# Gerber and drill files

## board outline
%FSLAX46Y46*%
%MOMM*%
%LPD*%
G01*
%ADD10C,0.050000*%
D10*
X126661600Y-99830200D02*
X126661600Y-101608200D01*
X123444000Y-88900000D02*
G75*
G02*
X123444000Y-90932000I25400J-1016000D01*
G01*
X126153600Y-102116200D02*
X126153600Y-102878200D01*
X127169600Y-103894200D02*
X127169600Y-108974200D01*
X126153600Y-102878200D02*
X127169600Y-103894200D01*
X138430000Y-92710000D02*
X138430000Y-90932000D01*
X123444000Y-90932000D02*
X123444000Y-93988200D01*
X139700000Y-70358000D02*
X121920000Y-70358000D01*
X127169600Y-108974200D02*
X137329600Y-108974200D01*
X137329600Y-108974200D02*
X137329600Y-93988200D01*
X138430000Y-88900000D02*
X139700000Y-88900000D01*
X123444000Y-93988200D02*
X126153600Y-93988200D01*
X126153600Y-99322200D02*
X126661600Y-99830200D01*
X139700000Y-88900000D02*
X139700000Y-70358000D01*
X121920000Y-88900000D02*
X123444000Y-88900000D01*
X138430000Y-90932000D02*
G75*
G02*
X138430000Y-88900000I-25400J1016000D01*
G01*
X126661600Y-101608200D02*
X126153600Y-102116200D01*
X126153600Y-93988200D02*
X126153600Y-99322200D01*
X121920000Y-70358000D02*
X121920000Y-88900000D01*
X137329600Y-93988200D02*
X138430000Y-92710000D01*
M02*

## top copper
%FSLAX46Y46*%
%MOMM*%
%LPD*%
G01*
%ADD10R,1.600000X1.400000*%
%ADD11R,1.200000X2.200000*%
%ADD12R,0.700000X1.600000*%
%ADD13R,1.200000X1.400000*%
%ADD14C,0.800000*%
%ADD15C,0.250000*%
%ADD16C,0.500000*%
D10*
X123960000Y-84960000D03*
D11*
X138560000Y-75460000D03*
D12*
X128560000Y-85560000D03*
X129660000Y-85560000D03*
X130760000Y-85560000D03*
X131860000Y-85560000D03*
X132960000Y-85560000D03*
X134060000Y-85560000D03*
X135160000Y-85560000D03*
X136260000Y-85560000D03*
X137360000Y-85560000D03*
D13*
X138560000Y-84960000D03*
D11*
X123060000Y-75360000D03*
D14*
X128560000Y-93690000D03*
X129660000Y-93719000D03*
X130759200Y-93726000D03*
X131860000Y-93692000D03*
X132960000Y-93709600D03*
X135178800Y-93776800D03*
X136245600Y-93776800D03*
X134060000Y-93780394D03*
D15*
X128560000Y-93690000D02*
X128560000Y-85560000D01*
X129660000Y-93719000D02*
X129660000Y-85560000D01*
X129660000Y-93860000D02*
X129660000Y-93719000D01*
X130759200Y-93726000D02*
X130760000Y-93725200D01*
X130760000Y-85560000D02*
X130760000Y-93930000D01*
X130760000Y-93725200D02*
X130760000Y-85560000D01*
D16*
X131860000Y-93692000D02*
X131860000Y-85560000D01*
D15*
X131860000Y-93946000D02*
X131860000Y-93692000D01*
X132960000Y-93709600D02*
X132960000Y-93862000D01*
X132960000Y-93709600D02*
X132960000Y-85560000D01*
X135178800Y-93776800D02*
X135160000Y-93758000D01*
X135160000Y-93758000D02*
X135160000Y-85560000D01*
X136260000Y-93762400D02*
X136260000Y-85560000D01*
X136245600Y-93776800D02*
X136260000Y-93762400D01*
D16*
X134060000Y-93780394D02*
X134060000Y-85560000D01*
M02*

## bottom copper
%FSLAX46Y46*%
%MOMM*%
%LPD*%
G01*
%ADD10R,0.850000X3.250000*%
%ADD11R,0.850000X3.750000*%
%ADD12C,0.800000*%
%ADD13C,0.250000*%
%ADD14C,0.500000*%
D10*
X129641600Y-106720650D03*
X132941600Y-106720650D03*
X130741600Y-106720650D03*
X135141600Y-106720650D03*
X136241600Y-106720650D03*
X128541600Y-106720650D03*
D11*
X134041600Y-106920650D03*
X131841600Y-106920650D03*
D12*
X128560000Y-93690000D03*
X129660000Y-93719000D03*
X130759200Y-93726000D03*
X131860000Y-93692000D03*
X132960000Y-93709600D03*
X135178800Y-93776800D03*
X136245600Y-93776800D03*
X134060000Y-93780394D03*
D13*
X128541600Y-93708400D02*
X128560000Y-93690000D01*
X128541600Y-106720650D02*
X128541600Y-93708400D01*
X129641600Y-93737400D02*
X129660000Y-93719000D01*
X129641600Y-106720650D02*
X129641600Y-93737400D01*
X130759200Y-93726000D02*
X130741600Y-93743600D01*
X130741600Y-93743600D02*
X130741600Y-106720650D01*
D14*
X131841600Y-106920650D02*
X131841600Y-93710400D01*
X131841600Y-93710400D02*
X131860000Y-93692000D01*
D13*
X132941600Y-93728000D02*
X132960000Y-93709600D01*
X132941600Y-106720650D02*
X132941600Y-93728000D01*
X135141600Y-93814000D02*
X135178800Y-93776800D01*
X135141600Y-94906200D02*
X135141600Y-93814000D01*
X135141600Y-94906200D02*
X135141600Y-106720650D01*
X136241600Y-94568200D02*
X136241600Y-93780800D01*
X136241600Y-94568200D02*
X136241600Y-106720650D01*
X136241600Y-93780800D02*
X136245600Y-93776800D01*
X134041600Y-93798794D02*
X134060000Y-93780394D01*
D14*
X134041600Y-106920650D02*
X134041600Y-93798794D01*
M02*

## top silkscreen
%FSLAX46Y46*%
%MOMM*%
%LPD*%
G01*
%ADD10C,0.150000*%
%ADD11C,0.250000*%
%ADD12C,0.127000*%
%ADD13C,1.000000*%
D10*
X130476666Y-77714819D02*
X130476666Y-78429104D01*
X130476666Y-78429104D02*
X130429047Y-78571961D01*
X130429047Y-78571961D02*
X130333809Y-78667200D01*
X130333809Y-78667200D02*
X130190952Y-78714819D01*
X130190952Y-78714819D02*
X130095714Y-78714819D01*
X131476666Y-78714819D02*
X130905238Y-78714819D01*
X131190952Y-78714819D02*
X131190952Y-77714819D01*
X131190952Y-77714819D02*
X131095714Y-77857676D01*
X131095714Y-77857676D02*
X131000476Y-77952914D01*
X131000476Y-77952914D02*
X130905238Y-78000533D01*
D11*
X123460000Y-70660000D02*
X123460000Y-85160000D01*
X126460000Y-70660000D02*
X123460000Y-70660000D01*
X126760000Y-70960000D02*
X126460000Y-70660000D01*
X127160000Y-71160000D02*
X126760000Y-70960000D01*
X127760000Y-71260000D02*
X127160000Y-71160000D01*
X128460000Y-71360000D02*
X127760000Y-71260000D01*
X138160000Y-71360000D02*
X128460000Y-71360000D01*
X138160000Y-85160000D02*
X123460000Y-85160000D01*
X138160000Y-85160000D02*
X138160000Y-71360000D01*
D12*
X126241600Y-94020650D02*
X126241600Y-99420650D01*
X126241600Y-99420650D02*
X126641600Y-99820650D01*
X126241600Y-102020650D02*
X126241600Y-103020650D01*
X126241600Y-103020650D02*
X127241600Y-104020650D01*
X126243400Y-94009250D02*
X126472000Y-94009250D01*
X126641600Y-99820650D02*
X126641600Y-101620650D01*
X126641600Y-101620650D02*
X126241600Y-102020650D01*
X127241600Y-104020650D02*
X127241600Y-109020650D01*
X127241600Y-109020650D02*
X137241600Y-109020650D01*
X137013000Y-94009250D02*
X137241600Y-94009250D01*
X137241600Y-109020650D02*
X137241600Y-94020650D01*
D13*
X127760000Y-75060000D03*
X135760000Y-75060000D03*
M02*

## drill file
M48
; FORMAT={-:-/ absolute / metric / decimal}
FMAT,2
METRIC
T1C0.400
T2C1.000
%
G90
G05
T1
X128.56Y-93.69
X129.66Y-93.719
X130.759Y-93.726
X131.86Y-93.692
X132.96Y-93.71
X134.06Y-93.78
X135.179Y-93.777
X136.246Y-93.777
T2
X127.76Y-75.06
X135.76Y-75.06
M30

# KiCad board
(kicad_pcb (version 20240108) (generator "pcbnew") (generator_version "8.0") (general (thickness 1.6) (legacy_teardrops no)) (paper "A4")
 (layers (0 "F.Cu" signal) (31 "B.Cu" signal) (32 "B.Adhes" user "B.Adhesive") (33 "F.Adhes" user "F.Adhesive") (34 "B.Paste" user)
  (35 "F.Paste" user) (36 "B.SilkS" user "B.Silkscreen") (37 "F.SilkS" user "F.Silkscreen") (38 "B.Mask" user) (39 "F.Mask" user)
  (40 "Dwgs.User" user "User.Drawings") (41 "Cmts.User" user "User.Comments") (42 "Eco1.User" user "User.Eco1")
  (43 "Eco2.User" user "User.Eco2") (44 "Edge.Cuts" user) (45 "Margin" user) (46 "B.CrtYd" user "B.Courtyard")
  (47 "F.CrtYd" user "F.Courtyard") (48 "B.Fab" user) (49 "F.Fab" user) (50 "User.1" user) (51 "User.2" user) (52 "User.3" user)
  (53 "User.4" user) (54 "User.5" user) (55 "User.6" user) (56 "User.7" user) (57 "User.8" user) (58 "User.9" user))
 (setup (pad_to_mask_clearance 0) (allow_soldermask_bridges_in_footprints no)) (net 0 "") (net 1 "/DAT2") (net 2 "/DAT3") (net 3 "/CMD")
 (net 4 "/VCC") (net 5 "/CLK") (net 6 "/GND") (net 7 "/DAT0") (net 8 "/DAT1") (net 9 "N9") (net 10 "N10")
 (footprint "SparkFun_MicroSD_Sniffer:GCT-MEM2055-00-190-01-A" (layer "F.Cu") (at 130.81 86.36)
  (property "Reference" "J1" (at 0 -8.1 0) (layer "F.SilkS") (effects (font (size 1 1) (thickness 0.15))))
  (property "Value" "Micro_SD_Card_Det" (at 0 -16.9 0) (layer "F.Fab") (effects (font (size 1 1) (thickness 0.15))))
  (fp_line (start -7.35 -15.7) (end -7.35 -1.2) (stroke (width 0.25) (type solid)) (layer "F.SilkS"))
  (fp_line (start -4.35 -15.7) (end -7.35 -15.7) (stroke (width 0.25) (type solid)) (layer "F.SilkS"))
  (fp_line (start -4.05 -15.4) (end -4.35 -15.7) (stroke (width 0.25) (type solid)) (layer "F.SilkS"))
  (fp_line (start -3.65 -15.2) (end -4.05 -15.4) (stroke (width 0.25) (type solid)) (layer "F.SilkS"))
  (fp_line (start -3.05 -15.1) (end -3.65 -15.2) (stroke (width 0.25) (type solid)) (layer "F.SilkS"))
  (fp_line (start -2.35 -15) (end -3.05 -15.1) (stroke (width 0.25) (type solid)) (layer "F.SilkS"))
  (fp_line (start 7.35 -15) (end -2.35 -15) (stroke (width 0.25) (type solid)) (layer "F.SilkS"))
  (fp_line (start 7.35 -1.2) (end -7.35 -1.2) (stroke (width 0.25) (type solid)) (layer "F.SilkS"))
  (fp_line (start 7.35 -1.2) (end 7.35 -15) (stroke (width 0.25) (type solid)) (layer "F.SilkS"))
  (pad "" smd rect (at -6.85 -1.4) (size 1.6 1.4) (layers "F.Cu" "F.Paste" "F.Mask"))
  (pad "" np_thru_hole circle (at -3.05 -11.3 180) (size 1 1) (drill 1) (layers "*.Cu" "*.Mask" "F.SilkS"))
  (pad "" np_thru_hole circle (at 4.95 -11.3 180) (size 1 1) (drill 1) (layers "*.Cu" "*.Mask" "F.SilkS"))
  (pad "" smd rect (at 7.75 -10.9 180) (size 1.2 2.2) (layers "F.Cu" "F.Paste" "F.Mask"))
  (pad "1" smd rect (at -2.25 -0.8) (size 0.7 1.6) (layers "F.Cu" "F.Paste" "F.Mask") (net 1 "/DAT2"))
  (pad "2" smd rect (at -1.15 -0.8) (size 0.7 1.6) (layers "F.Cu" "F.Paste" "F.Mask") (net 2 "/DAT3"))
  (pad "3" smd rect (at -0.05 -0.8) (size 0.7 1.6) (layers "F.Cu" "F.Paste" "F.Mask") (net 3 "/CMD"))
  (pad "4" smd rect (at 1.05 -0.8) (size 0.7 1.6) (layers "F.Cu" "F.Paste" "F.Mask") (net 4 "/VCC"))
  (pad "5" smd rect (at 2.15 -0.8) (size 0.7 1.6) (layers "F.Cu" "F.Paste" "F.Mask") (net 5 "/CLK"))
  (pad "6" smd rect (at 3.25 -0.8) (size 0.7 1.6) (layers "F.Cu" "F.Paste" "F.Mask") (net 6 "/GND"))
  (pad "7" smd rect (at 4.35 -0.8) (size 0.7 1.6) (layers "F.Cu" "F.Paste" "F.Mask") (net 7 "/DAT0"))
  (pad "8" smd rect (at 5.45 -0.8) (size 0.7 1.6) (layers "F.Cu" "F.Paste" "F.Mask") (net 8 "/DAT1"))
  (pad "9" smd rect (at 6.55 -0.8) (size 0.7 1.6) (layers "F.Cu" "F.Paste" "F.Mask") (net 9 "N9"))
  (pad "10" smd rect (at 7.75 -1.4) (size 1.2 1.4) (layers "F.Cu" "F.Paste" "F.Mask") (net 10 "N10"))
  (pad "~" smd rect (at -7.75 -11 180) (size 1.2 2.2) (layers "F.Cu" "F.Paste" "F.Mask")))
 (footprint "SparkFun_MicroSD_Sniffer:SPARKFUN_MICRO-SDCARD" (layer "F.Cu") (at 127.0816 109.02065)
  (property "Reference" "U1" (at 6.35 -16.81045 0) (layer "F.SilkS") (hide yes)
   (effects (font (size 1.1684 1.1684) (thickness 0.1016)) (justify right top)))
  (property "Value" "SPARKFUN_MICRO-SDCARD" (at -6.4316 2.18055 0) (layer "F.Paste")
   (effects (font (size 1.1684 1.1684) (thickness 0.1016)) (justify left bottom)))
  (fp_line (start -0.84 -15) (end -0.84 -9.6) (stroke (width 0.127) (type solid)) (layer "F.SilkS"))
  (fp_line (start -0.84 -9.6) (end -0.44 -9.2) (stroke (width 0.127) (type solid)) (layer "F.SilkS"))
  (fp_line (start -0.84 -7) (end -0.84 -6) (stroke (width 0.127) (type solid)) (layer "F.SilkS"))
  (fp_line (start -0.84 -6) (end 0.16 -5) (stroke (width 0.127) (type solid)) (layer "F.SilkS"))
  (fp_line (start -0.8382 -15.0114) (end -0.6096 -15.0114) (stroke (width 0.127) (type solid)) (layer "F.SilkS"))
  (fp_line (start -0.44 -9.2) (end -0.44 -7.4) (stroke (width 0.127) (type solid)) (layer "F.SilkS"))
  (fp_line (start -0.44 -7.4) (end -0.84 -7) (stroke (width 0.127) (type solid)) (layer "F.SilkS"))
  (fp_line (start 0.16 -5) (end 0.16 0) (stroke (width 0.127) (type solid)) (layer "F.SilkS"))
  (fp_line (start 0.16 0) (end 10.16 0) (stroke (width 0.127) (type solid)) (layer "F.SilkS"))
  (fp_line (start 9.9314 -15.0114) (end 10.16 -15.0114) (stroke (width 0.127) (type solid)) (layer "F.SilkS"))
  (fp_line (start 10.16 0) (end 10.16 -15) (stroke (width 0.127) (type solid)) (layer "F.SilkS"))
  (pad "CD/DAT3" smd rect (at 2.56 -2.3) (size 0.85 3.25) (layers "B.Cu" "B.Paste" "B.Mask") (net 2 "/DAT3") (solder_mask_margin 0.1016))
  (pad "CLK" smd rect (at 5.86 -2.3) (size 0.85 3.25) (layers "B.Cu" "B.Paste" "B.Mask") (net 5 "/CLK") (solder_mask_margin 0.1016))
  (pad "CMD" smd rect (at 3.66 -2.3) (size 0.85 3.25) (layers "B.Cu" "B.Paste" "B.Mask") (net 3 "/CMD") (solder_mask_margin 0.1016))
  (pad "DAT0" smd rect (at 8.06 -2.3) (size 0.85 3.25) (layers "B.Cu" "B.Paste" "B.Mask") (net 7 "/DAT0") (solder_mask_margin 0.1016))
  (pad "DAT1" smd rect (at 9.16 -2.3) (size 0.85 3.25) (layers "B.Cu" "B.Paste" "B.Mask") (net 8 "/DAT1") (solder_mask_margin 0.1016))
  (pad "DAT2" smd rect (at 1.46 -2.3) (size 0.85 3.25) (layers "B.Cu" "B.Paste" "B.Mask") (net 1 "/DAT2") (solder_mask_margin 0.1016))
  (pad "GND" smd rect (at 6.96 -2.1 180) (size 0.85 3.75) (layers "B.Cu" "B.Paste" "B.Mask") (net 6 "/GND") (solder_mask_margin 0.1016))
  (pad "VCC" smd rect (at 4.76 -2.1) (size 0.85 3.75) (layers "B.Cu" "B.Paste" "B.Mask") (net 4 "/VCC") (solder_mask_margin 0.1016)))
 (gr_line (start 126.6616 99.8302) (end 126.6616 101.6082) (stroke (width 0.05) (type solid)) (layer "Edge.Cuts"))
 (gr_arc (start 123.444 88.9) (mid 124.485717 89.916) (end 123.444 90.932) (stroke (width 0.05) (type solid)) (layer "Edge.Cuts"))
 (gr_line (start 126.1536 102.1162) (end 126.1536 102.8782) (stroke (width 0.05) (type solid)) (layer "Edge.Cuts"))
 (gr_line (start 127.1696 103.8942) (end 127.1696 108.9742) (stroke (width 0.05) (type solid)) (layer "Edge.Cuts"))
 (gr_line (start 126.1536 102.8782) (end 127.1696 103.8942) (stroke (width 0.05) (type solid)) (layer "Edge.Cuts"))
 (gr_line (start 138.43 92.71) (end 138.43 90.932) (stroke (width 0.05) (type solid)) (layer "Edge.Cuts"))
 (gr_line (start 123.444 90.932) (end 123.444 93.9882) (stroke (width 0.05) (type solid)) (layer "Edge.Cuts"))
 (gr_line (start 139.7 70.358) (end 121.92 70.358) (stroke (width 0.05) (type solid)) (layer "Edge.Cuts"))
 (gr_line (start 127.1696 108.9742) (end 137.3296 108.9742) (stroke (width 0.05) (type solid)) (layer "Edge.Cuts"))
 (gr_line (start 137.3296 108.9742) (end 137.3296 93.9882) (stroke (width 0.05) (type solid)) (layer "Edge.Cuts"))
 (gr_line (start 138.43 88.9) (end 139.7 88.9) (stroke (width 0.05) (type solid)) (layer "Edge.Cuts"))
 (gr_line (start 123.444 93.9882) (end 126.1536 93.9882) (stroke (width 0.05) (type solid)) (layer "Edge.Cuts"))
 (gr_line (start 126.1536 99.3222) (end 126.6616 99.8302) (stroke (width 0.05) (type solid)) (layer "Edge.Cuts"))
 (gr_line (start 139.7 88.9) (end 139.7 70.358) (stroke (width 0.05) (type solid)) (layer "Edge.Cuts"))
 (gr_line (start 121.92 88.9) (end 123.444 88.9) (stroke (width 0.05) (type solid)) (layer "Edge.Cuts"))
 (gr_arc (start 138.43 90.932) (mid 137.388283 89.916) (end 138.43 88.9) (stroke (width 0.05) (type solid)) (layer "Edge.Cuts"))
 (gr_line (start 126.6616 101.6082) (end 126.1536 102.1162) (stroke (width 0.05) (type solid)) (layer "Edge.Cuts"))
 (gr_line (start 126.1536 93.9882) (end 126.1536 99.3222) (stroke (width 0.05) (type solid)) (layer "Edge.Cuts"))
 (gr_line (start 121.92 70.358) (end 121.92 88.9) (stroke (width 0.05) (type solid)) (layer "Edge.Cuts"))
 (gr_line (start 137.3296 93.9882) (end 138.43 92.71) (stroke (width 0.05) (type solid)) (layer "Edge.Cuts"))
 (segment (start 128.56 93.69) (end 128.56 85.56) (width 0.25) (layer "F.Cu") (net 1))
 (via (at 128.56 93.69) (size 0.8) (drill 0.4) (layers "F.Cu" "B.Cu") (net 1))
 (segment (start 128.5416 93.7084) (end 128.56 93.69) (width 0.25) (layer "B.Cu") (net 1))
 (segment (start 128.5416 106.72065) (end 128.5416 93.7084) (width 0.25) (layer "B.Cu") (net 1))
 (segment (start 129.66 93.719) (end 129.66 85.56) (width 0.25) (layer "F.Cu") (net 2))
 (segment (start 129.66 93.86) (end 129.66 93.719) (width 0.25) (layer "F.Cu") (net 2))
 (via (at 129.66 93.719) (size 0.8) (drill 0.4) (layers "F.Cu" "B.Cu") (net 2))
 (segment (start 129.6416 93.7374) (end 129.66 93.719) (width 0.25) (layer "B.Cu") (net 2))
 (segment (start 129.6416 106.72065) (end 129.6416 93.7374) (width 0.25) (layer "B.Cu") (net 2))
 (segment (start 130.7592 93.726) (end 130.76 93.7252) (width 0.25) (layer "F.Cu") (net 3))
 (segment (start 130.76 85.56) (end 130.76 93.93) (width 0.25) (layer "F.Cu") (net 3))
 (segment (start 130.76 93.7252) (end 130.76 85.56) (width 0.25) (layer "F.Cu") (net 3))
 (via (at 130.7592 93.726) (size 0.8) (drill 0.4) (layers "F.Cu" "B.Cu") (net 3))
 (segment (start 130.7592 93.726) (end 130.7416 93.7436) (width 0.25) (layer "B.Cu") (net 3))
 (segment (start 130.7416 93.7436) (end 130.7416 106.72065) (width 0.25) (layer "B.Cu") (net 3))
 (segment (start 131.86 93.692) (end 131.86 85.56) (width 0.5) (layer "F.Cu") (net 4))
 (segment (start 131.86 93.946) (end 131.86 93.692) (width 0.25) (layer "F.Cu") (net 4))
 (via (at 131.86 93.692) (size 0.8) (drill 0.4) (layers "F.Cu" "B.Cu") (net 4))
 (segment (start 131.8416 106.92065) (end 131.8416 93.7104) (width 0.5) (layer "B.Cu") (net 4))
 (segment (start 131.8416 93.7104) (end 131.86 93.692) (width 0.5) (layer "B.Cu") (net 4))
 (segment (start 132.96 93.7096) (end 132.96 93.862) (width 0.25) (layer "F.Cu") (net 5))
 (segment (start 132.96 93.7096) (end 132.96 85.56) (width 0.25) (layer "F.Cu") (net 5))
 (via (at 132.96 93.7096) (size 0.8) (drill 0.4) (layers "F.Cu" "B.Cu") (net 5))
 (segment (start 132.9416 93.728) (end 132.96 93.7096) (width 0.25) (layer "B.Cu") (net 5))
 (segment (start 132.9416 106.72065) (end 132.9416 93.728) (width 0.25) (layer "B.Cu") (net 5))
 (segment (start 135.1788 93.7768) (end 135.16 93.758) (width 0.25) (layer "F.Cu") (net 7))
 (segment (start 135.16 93.758) (end 135.16 85.56) (width 0.25) (layer "F.Cu") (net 7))
 (via (at 135.1788 93.7768) (size 0.8) (drill 0.4) (layers "F.Cu" "B.Cu") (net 7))
 (segment (start 135.1416 93.814) (end 135.1788 93.7768) (width 0.25) (layer "B.Cu") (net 7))
 (segment (start 135.1416 94.9062) (end 135.1416 93.814) (width 0.25) (layer "B.Cu") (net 7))
 (segment (start 135.1416 94.9062) (end 135.1416 106.72065) (width 0.25) (layer "B.Cu") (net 7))
 (segment (start 136.26 93.7624) (end 136.26 85.56) (width 0.25) (layer "F.Cu") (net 8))
 (segment (start 136.2456 93.7768) (end 136.26 93.7624) (width 0.25) (layer "F.Cu") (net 8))
 (via (at 136.2456 93.7768) (size 0.8) (drill 0.4) (layers "F.Cu" "B.Cu") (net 8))
 (segment (start 136.2416 94.5682) (end 136.2416 93.7808) (width 0.25) (layer "B.Cu") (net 8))
 (segment (start 136.2416 94.5682) (end 136.2416 106.72065) (width 0.25) (layer "B.Cu") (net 8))
 (segment (start 136.2416 93.7808) (end 136.2456 93.7768) (width 0.25) (layer "B.Cu") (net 8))
 (segment (start 134.06 93.780394) (end 134.06 85.56) (width 0.5) (layer "F.Cu") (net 6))
 (via (at 134.06 93.780394) (size 0.8) (drill 0.4) (layers "F.Cu" "B.Cu") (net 6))
 (segment (start 134.0416 93.798794) (end 134.06 93.780394) (width 0.25) (layer "B.Cu") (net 6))
 (segment (start 134.0416 106.92065) (end 134.0416 93.798794) (width 0.5) (layer "B.Cu") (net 6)))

